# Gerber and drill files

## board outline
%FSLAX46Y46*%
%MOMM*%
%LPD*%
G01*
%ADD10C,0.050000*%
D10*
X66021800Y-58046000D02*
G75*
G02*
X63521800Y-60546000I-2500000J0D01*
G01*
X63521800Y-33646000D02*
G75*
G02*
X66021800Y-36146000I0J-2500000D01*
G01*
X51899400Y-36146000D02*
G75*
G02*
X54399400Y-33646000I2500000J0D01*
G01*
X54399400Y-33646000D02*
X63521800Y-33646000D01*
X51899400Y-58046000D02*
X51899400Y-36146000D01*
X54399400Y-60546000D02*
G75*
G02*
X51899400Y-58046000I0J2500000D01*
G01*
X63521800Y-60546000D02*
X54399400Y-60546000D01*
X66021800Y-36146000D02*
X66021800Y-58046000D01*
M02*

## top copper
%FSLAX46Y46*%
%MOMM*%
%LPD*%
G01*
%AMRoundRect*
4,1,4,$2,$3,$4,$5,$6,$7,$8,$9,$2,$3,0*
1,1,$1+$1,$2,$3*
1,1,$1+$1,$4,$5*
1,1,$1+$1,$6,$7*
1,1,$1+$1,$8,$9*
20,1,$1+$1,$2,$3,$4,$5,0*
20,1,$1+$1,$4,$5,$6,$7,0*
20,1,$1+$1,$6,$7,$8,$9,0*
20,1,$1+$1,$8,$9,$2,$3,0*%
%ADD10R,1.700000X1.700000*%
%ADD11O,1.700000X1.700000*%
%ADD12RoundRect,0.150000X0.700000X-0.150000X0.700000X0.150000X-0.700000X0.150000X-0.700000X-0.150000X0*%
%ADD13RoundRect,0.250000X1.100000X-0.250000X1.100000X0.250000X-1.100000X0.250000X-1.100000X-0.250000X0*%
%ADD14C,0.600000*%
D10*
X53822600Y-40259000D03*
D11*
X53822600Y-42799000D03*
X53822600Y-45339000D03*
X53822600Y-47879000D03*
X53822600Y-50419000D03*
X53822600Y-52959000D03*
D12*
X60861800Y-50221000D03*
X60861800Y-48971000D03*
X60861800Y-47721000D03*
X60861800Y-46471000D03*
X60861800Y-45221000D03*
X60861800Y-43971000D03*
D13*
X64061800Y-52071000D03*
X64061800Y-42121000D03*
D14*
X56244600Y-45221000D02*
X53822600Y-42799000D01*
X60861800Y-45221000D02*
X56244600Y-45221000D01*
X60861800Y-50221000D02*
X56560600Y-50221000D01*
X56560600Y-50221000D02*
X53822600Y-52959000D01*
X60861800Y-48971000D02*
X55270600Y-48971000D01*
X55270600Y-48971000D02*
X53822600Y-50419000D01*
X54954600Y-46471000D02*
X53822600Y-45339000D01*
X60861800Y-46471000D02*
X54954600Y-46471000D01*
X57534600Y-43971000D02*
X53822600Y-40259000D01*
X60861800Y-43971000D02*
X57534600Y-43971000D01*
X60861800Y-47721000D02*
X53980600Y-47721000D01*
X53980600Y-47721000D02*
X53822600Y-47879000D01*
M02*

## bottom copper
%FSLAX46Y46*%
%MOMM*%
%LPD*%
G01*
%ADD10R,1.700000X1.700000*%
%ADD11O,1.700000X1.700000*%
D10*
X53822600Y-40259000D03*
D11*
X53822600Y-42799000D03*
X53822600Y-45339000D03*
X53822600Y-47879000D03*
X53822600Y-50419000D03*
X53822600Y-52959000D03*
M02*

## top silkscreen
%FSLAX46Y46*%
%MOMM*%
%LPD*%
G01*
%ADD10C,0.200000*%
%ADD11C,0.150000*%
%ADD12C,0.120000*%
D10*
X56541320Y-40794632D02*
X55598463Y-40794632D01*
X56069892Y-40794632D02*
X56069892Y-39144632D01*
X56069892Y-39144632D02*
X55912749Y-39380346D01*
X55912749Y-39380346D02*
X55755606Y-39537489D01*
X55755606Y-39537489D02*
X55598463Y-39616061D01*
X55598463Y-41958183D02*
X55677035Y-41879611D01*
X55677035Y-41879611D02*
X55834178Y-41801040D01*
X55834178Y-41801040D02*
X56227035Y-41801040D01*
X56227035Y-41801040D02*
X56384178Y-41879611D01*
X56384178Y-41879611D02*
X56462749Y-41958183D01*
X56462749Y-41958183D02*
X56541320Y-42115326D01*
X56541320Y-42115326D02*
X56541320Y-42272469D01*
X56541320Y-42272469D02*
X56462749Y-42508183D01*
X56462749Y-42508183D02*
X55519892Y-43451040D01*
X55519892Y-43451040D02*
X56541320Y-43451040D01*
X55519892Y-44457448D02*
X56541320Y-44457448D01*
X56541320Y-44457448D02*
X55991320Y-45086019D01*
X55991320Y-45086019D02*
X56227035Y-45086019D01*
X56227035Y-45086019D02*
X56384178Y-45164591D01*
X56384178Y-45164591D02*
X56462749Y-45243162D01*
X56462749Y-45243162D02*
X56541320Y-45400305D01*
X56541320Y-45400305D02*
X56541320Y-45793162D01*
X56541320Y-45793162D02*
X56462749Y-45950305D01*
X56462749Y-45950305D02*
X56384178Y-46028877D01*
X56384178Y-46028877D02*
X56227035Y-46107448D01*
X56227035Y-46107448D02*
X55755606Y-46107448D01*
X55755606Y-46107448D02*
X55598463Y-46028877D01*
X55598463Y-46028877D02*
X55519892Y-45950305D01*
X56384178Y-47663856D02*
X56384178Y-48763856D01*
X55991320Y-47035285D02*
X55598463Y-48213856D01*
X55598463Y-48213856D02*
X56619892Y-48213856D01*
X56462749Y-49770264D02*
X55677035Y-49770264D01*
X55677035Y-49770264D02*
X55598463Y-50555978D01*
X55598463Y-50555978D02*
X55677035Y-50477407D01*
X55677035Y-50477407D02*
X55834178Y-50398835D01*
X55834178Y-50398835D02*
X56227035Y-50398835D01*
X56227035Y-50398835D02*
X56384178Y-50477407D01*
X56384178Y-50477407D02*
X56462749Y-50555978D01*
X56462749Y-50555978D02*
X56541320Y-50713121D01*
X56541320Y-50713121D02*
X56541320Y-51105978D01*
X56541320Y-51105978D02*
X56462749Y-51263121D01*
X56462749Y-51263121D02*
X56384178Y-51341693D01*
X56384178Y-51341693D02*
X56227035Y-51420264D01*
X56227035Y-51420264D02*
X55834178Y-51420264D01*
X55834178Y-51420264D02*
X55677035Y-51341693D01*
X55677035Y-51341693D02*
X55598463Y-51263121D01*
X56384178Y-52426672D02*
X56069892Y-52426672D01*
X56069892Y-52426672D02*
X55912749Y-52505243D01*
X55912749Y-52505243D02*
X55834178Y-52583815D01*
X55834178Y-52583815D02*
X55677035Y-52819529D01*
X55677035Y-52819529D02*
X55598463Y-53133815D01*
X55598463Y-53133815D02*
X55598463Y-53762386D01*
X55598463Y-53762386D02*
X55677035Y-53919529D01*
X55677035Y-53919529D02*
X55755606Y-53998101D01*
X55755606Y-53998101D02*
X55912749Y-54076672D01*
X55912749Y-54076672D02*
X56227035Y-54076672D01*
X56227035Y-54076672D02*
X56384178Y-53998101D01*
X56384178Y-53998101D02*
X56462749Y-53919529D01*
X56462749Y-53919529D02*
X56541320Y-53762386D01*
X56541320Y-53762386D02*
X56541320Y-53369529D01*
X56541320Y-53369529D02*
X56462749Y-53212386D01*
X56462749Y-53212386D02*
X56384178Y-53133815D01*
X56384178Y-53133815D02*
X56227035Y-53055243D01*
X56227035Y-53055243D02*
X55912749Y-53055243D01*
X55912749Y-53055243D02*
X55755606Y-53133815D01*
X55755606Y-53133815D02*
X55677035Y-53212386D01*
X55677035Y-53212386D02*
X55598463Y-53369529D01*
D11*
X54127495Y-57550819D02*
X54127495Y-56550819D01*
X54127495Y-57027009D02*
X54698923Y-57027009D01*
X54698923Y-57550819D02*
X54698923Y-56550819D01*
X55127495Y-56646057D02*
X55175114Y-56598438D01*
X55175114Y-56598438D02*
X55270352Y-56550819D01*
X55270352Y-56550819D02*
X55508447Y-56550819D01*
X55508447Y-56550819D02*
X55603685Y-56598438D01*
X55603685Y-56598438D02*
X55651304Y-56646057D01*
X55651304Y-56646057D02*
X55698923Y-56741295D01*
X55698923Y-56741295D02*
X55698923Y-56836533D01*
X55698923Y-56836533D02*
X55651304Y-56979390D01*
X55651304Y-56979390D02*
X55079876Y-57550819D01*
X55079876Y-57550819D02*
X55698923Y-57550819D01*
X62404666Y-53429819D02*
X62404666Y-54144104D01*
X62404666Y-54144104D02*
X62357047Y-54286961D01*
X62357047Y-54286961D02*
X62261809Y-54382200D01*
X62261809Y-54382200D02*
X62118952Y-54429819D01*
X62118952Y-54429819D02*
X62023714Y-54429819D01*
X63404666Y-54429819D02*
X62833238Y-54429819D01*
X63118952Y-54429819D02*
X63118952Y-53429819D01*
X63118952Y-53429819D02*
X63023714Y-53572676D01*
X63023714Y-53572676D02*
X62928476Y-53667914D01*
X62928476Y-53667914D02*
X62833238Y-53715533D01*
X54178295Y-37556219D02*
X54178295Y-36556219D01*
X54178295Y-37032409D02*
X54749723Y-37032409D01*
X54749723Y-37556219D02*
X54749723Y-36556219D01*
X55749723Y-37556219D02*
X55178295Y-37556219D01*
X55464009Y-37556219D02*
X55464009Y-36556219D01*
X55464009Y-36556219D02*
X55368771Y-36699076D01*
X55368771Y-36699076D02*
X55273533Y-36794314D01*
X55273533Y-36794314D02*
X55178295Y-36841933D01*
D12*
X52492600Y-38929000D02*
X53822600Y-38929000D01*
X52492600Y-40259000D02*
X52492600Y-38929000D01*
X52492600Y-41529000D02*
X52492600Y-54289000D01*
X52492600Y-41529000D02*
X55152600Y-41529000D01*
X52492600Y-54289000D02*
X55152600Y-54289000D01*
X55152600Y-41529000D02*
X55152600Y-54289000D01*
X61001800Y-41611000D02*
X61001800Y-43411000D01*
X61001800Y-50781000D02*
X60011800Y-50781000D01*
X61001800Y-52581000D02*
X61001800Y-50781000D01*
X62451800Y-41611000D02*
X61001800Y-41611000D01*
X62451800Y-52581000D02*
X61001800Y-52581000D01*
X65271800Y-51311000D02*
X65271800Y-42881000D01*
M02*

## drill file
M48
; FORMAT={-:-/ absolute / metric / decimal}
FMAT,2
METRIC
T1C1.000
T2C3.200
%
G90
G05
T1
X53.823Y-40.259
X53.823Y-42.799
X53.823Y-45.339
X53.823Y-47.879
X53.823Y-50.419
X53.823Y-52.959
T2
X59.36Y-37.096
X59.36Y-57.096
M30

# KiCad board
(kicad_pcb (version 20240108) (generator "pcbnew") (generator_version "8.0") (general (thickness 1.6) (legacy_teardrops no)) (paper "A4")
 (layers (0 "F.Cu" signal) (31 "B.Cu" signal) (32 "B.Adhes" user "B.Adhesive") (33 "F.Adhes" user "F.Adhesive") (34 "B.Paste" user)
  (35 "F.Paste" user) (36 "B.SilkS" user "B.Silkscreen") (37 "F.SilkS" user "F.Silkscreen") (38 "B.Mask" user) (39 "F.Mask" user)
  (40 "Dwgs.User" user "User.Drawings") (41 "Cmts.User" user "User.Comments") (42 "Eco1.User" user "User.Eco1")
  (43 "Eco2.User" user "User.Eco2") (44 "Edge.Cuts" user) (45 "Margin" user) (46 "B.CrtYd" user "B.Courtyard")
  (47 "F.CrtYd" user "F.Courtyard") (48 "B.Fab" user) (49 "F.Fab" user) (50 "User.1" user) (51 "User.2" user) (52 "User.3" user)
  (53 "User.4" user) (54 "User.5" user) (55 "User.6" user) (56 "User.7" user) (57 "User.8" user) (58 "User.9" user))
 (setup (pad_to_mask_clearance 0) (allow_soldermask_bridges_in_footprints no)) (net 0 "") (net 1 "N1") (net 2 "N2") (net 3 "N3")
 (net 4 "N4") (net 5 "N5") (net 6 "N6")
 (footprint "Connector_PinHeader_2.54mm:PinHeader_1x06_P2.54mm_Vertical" (layer "F.Cu") (at 53.8226 40.259)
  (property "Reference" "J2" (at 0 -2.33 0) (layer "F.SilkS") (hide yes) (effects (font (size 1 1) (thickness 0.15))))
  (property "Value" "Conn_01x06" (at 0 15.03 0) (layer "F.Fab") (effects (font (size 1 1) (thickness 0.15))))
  (fp_line (start -1.33 -1.33) (end 0 -1.33) (stroke (width 0.12) (type solid)) (layer "F.SilkS"))
  (fp_line (start -1.33 0) (end -1.33 -1.33) (stroke (width 0.12) (type solid)) (layer "F.SilkS"))
  (fp_line (start -1.33 1.27) (end -1.33 14.03) (stroke (width 0.12) (type solid)) (layer "F.SilkS"))
  (fp_line (start -1.33 1.27) (end 1.33 1.27) (stroke (width 0.12) (type solid)) (layer "F.SilkS"))
  (fp_line (start -1.33 14.03) (end 1.33 14.03) (stroke (width 0.12) (type solid)) (layer "F.SilkS"))
  (fp_line (start 1.33 1.27) (end 1.33 14.03) (stroke (width 0.12) (type solid)) (layer "F.SilkS"))
  (pad "1" thru_hole rect (at 0 0) (size 1.7 1.7) (drill 1) (layers "*.Cu" "*.Mask") (remove_unused_layers no) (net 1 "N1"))
  (pad "2" thru_hole oval (at 0 2.54) (size 1.7 1.7) (drill 1) (layers "*.Cu" "*.Mask") (remove_unused_layers no) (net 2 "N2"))
  (pad "3" thru_hole oval (at 0 5.08) (size 1.7 1.7) (drill 1) (layers "*.Cu" "*.Mask") (remove_unused_layers no) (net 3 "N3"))
  (pad "4" thru_hole oval (at 0 7.62) (size 1.7 1.7) (drill 1) (layers "*.Cu" "*.Mask") (remove_unused_layers no) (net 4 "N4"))
  (pad "5" thru_hole oval (at 0 10.16) (size 1.7 1.7) (drill 1) (layers "*.Cu" "*.Mask") (remove_unused_layers no) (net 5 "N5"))
  (pad "6" thru_hole oval (at 0 12.7) (size 1.7 1.7) (drill 1) (layers "*.Cu" "*.Mask") (remove_unused_layers no) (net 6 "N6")))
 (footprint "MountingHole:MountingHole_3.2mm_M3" (layer "F.Cu") (at 59.3598 57.096)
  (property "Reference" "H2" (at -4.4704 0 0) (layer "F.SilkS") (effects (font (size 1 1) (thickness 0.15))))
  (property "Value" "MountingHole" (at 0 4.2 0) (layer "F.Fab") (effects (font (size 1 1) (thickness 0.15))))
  (pad "" np_thru_hole circle (at 0 0) (size 3.2 3.2) (drill 3.2) (layers "*.Cu" "*.Mask")))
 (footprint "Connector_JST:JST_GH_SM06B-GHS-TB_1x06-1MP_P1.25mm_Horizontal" (layer "F.Cu") (at 62.7118 47.096 90)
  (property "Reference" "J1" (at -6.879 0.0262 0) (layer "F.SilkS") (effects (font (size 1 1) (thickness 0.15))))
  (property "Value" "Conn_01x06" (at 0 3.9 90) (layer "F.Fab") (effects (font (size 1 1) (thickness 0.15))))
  (fp_line (start 5.485 -1.71) (end 3.685 -1.71) (stroke (width 0.12) (type solid)) (layer "F.SilkS"))
  (fp_line (start -3.685 -1.71) (end -3.685 -2.7) (stroke (width 0.12) (type solid)) (layer "F.SilkS"))
  (fp_line (start -5.485 -1.71) (end -3.685 -1.71) (stroke (width 0.12) (type solid)) (layer "F.SilkS"))
  (fp_line (start 5.485 -0.26) (end 5.485 -1.71) (stroke (width 0.12) (type solid)) (layer "F.SilkS"))
  (fp_line (start -5.485 -0.26) (end -5.485 -1.71) (stroke (width 0.12) (type solid)) (layer "F.SilkS"))
  (fp_line (start -4.215 2.56) (end 4.215 2.56) (stroke (width 0.12) (type solid)) (layer "F.SilkS"))
  (pad "1" smd roundrect (at -3.125 -1.85 90) (size 0.6 1.7) (layers "F.Cu" "F.Paste" "F.Mask") (roundrect_rratio 0.25) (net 6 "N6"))
  (pad "2" smd roundrect (at -1.875 -1.85 90) (size 0.6 1.7) (layers "F.Cu" "F.Paste" "F.Mask") (roundrect_rratio 0.25) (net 5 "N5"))
  (pad "3" smd roundrect (at -0.625 -1.85 90) (size 0.6 1.7) (layers "F.Cu" "F.Paste" "F.Mask") (roundrect_rratio 0.25) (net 4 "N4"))
  (pad "4" smd roundrect (at 0.625 -1.85 90) (size 0.6 1.7) (layers "F.Cu" "F.Paste" "F.Mask") (roundrect_rratio 0.25) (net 3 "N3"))
  (pad "5" smd roundrect (at 1.875 -1.85 90) (size 0.6 1.7) (layers "F.Cu" "F.Paste" "F.Mask") (roundrect_rratio 0.25) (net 2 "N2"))
  (pad "6" smd roundrect (at 3.125 -1.85 90) (size 0.6 1.7) (layers "F.Cu" "F.Paste" "F.Mask") (roundrect_rratio 0.25) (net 1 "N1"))
  (pad "MP" smd roundrect (at -4.975 1.35 90) (size 1 2.7) (layers "F.Cu" "F.Paste" "F.Mask") (roundrect_rratio 0.25))
  (pad "MP" smd roundrect (at 4.975 1.35 90) (size 1 2.7) (layers "F.Cu" "F.Paste" "F.Mask") (roundrect_rratio 0.25)))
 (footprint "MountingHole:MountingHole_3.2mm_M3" (layer "F.Cu") (at 59.3598 37.096)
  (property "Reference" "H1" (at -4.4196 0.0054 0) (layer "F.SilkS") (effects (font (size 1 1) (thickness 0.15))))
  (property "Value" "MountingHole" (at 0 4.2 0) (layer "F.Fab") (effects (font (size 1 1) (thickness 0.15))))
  (pad "" np_thru_hole circle (at 0 0) (size 3.2 3.2) (drill 3.2) (layers "*.Cu" "*.Mask")))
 (gr_arc (start 66.0218 58.046) (mid 65.289567 59.813767) (end 63.5218 60.546) (stroke (width 0.05) (type default)) (layer "Edge.Cuts"))
 (gr_arc (start 63.5218 33.646) (mid 65.289567 34.378233) (end 66.0218 36.146) (stroke (width 0.05) (type default)) (layer "Edge.Cuts"))
 (gr_arc (start 51.8994 36.146) (mid 52.631633 34.378233) (end 54.3994 33.646) (stroke (width 0.05) (type default)) (layer "Edge.Cuts"))
 (gr_line (start 54.3994 33.646) (end 63.5218 33.646) (stroke (width 0.05) (type default)) (layer "Edge.Cuts"))
 (gr_line (start 51.8994 58.046) (end 51.8994 36.146) (stroke (width 0.05) (type default)) (layer "Edge.Cuts"))
 (gr_arc (start 54.3994 60.546) (mid 52.631633 59.813767) (end 51.8994 58.046) (stroke (width 0.05) (type default)) (layer "Edge.Cuts"))
 (gr_line (start 63.5218 60.546) (end 54.3994 60.546) (stroke (width 0.05) (type default)) (layer "Edge.Cuts"))
 (gr_line (start 66.0218 36.146) (end 66.0218 58.046) (stroke (width 0.05) (type default)) (layer "Edge.Cuts"))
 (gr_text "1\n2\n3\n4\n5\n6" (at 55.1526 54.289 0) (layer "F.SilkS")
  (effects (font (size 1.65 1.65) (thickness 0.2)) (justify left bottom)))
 (segment (start 56.2446 45.221) (end 53.8226 42.799) (width 0.6) (layer "F.Cu") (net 2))
 (segment (start 60.8618 45.221) (end 56.2446 45.221) (width 0.6) (layer "F.Cu") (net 2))
 (segment (start 60.8618 50.221) (end 56.5606 50.221) (width 0.6) (layer "F.Cu") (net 6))
 (segment (start 56.5606 50.221) (end 53.8226 52.959) (width 0.6) (layer "F.Cu") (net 6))
 (segment (start 60.8618 48.971) (end 55.2706 48.971) (width 0.6) (layer "F.Cu") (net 5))
 (segment (start 55.2706 48.971) (end 53.8226 50.419) (width 0.6) (layer "F.Cu") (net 5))
 (segment (start 54.9546 46.471) (end 53.8226 45.339) (width 0.6) (layer "F.Cu") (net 3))
 (segment (start 60.8618 46.471) (end 54.9546 46.471) (width 0.6) (layer "F.Cu") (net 3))
 (segment (start 57.5346 43.971) (end 53.8226 40.259) (width 0.6) (layer "F.Cu") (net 1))
 (segment (start 60.8618 43.971) (end 57.5346 43.971) (width 0.6) (layer "F.Cu") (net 1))
 (segment (start 60.8618 47.721) (end 53.9806 47.721) (width 0.6) (layer "F.Cu") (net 4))
 (segment (start 53.9806 47.721) (end 53.8226 47.879) (width 0.6) (layer "F.Cu") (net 4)))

